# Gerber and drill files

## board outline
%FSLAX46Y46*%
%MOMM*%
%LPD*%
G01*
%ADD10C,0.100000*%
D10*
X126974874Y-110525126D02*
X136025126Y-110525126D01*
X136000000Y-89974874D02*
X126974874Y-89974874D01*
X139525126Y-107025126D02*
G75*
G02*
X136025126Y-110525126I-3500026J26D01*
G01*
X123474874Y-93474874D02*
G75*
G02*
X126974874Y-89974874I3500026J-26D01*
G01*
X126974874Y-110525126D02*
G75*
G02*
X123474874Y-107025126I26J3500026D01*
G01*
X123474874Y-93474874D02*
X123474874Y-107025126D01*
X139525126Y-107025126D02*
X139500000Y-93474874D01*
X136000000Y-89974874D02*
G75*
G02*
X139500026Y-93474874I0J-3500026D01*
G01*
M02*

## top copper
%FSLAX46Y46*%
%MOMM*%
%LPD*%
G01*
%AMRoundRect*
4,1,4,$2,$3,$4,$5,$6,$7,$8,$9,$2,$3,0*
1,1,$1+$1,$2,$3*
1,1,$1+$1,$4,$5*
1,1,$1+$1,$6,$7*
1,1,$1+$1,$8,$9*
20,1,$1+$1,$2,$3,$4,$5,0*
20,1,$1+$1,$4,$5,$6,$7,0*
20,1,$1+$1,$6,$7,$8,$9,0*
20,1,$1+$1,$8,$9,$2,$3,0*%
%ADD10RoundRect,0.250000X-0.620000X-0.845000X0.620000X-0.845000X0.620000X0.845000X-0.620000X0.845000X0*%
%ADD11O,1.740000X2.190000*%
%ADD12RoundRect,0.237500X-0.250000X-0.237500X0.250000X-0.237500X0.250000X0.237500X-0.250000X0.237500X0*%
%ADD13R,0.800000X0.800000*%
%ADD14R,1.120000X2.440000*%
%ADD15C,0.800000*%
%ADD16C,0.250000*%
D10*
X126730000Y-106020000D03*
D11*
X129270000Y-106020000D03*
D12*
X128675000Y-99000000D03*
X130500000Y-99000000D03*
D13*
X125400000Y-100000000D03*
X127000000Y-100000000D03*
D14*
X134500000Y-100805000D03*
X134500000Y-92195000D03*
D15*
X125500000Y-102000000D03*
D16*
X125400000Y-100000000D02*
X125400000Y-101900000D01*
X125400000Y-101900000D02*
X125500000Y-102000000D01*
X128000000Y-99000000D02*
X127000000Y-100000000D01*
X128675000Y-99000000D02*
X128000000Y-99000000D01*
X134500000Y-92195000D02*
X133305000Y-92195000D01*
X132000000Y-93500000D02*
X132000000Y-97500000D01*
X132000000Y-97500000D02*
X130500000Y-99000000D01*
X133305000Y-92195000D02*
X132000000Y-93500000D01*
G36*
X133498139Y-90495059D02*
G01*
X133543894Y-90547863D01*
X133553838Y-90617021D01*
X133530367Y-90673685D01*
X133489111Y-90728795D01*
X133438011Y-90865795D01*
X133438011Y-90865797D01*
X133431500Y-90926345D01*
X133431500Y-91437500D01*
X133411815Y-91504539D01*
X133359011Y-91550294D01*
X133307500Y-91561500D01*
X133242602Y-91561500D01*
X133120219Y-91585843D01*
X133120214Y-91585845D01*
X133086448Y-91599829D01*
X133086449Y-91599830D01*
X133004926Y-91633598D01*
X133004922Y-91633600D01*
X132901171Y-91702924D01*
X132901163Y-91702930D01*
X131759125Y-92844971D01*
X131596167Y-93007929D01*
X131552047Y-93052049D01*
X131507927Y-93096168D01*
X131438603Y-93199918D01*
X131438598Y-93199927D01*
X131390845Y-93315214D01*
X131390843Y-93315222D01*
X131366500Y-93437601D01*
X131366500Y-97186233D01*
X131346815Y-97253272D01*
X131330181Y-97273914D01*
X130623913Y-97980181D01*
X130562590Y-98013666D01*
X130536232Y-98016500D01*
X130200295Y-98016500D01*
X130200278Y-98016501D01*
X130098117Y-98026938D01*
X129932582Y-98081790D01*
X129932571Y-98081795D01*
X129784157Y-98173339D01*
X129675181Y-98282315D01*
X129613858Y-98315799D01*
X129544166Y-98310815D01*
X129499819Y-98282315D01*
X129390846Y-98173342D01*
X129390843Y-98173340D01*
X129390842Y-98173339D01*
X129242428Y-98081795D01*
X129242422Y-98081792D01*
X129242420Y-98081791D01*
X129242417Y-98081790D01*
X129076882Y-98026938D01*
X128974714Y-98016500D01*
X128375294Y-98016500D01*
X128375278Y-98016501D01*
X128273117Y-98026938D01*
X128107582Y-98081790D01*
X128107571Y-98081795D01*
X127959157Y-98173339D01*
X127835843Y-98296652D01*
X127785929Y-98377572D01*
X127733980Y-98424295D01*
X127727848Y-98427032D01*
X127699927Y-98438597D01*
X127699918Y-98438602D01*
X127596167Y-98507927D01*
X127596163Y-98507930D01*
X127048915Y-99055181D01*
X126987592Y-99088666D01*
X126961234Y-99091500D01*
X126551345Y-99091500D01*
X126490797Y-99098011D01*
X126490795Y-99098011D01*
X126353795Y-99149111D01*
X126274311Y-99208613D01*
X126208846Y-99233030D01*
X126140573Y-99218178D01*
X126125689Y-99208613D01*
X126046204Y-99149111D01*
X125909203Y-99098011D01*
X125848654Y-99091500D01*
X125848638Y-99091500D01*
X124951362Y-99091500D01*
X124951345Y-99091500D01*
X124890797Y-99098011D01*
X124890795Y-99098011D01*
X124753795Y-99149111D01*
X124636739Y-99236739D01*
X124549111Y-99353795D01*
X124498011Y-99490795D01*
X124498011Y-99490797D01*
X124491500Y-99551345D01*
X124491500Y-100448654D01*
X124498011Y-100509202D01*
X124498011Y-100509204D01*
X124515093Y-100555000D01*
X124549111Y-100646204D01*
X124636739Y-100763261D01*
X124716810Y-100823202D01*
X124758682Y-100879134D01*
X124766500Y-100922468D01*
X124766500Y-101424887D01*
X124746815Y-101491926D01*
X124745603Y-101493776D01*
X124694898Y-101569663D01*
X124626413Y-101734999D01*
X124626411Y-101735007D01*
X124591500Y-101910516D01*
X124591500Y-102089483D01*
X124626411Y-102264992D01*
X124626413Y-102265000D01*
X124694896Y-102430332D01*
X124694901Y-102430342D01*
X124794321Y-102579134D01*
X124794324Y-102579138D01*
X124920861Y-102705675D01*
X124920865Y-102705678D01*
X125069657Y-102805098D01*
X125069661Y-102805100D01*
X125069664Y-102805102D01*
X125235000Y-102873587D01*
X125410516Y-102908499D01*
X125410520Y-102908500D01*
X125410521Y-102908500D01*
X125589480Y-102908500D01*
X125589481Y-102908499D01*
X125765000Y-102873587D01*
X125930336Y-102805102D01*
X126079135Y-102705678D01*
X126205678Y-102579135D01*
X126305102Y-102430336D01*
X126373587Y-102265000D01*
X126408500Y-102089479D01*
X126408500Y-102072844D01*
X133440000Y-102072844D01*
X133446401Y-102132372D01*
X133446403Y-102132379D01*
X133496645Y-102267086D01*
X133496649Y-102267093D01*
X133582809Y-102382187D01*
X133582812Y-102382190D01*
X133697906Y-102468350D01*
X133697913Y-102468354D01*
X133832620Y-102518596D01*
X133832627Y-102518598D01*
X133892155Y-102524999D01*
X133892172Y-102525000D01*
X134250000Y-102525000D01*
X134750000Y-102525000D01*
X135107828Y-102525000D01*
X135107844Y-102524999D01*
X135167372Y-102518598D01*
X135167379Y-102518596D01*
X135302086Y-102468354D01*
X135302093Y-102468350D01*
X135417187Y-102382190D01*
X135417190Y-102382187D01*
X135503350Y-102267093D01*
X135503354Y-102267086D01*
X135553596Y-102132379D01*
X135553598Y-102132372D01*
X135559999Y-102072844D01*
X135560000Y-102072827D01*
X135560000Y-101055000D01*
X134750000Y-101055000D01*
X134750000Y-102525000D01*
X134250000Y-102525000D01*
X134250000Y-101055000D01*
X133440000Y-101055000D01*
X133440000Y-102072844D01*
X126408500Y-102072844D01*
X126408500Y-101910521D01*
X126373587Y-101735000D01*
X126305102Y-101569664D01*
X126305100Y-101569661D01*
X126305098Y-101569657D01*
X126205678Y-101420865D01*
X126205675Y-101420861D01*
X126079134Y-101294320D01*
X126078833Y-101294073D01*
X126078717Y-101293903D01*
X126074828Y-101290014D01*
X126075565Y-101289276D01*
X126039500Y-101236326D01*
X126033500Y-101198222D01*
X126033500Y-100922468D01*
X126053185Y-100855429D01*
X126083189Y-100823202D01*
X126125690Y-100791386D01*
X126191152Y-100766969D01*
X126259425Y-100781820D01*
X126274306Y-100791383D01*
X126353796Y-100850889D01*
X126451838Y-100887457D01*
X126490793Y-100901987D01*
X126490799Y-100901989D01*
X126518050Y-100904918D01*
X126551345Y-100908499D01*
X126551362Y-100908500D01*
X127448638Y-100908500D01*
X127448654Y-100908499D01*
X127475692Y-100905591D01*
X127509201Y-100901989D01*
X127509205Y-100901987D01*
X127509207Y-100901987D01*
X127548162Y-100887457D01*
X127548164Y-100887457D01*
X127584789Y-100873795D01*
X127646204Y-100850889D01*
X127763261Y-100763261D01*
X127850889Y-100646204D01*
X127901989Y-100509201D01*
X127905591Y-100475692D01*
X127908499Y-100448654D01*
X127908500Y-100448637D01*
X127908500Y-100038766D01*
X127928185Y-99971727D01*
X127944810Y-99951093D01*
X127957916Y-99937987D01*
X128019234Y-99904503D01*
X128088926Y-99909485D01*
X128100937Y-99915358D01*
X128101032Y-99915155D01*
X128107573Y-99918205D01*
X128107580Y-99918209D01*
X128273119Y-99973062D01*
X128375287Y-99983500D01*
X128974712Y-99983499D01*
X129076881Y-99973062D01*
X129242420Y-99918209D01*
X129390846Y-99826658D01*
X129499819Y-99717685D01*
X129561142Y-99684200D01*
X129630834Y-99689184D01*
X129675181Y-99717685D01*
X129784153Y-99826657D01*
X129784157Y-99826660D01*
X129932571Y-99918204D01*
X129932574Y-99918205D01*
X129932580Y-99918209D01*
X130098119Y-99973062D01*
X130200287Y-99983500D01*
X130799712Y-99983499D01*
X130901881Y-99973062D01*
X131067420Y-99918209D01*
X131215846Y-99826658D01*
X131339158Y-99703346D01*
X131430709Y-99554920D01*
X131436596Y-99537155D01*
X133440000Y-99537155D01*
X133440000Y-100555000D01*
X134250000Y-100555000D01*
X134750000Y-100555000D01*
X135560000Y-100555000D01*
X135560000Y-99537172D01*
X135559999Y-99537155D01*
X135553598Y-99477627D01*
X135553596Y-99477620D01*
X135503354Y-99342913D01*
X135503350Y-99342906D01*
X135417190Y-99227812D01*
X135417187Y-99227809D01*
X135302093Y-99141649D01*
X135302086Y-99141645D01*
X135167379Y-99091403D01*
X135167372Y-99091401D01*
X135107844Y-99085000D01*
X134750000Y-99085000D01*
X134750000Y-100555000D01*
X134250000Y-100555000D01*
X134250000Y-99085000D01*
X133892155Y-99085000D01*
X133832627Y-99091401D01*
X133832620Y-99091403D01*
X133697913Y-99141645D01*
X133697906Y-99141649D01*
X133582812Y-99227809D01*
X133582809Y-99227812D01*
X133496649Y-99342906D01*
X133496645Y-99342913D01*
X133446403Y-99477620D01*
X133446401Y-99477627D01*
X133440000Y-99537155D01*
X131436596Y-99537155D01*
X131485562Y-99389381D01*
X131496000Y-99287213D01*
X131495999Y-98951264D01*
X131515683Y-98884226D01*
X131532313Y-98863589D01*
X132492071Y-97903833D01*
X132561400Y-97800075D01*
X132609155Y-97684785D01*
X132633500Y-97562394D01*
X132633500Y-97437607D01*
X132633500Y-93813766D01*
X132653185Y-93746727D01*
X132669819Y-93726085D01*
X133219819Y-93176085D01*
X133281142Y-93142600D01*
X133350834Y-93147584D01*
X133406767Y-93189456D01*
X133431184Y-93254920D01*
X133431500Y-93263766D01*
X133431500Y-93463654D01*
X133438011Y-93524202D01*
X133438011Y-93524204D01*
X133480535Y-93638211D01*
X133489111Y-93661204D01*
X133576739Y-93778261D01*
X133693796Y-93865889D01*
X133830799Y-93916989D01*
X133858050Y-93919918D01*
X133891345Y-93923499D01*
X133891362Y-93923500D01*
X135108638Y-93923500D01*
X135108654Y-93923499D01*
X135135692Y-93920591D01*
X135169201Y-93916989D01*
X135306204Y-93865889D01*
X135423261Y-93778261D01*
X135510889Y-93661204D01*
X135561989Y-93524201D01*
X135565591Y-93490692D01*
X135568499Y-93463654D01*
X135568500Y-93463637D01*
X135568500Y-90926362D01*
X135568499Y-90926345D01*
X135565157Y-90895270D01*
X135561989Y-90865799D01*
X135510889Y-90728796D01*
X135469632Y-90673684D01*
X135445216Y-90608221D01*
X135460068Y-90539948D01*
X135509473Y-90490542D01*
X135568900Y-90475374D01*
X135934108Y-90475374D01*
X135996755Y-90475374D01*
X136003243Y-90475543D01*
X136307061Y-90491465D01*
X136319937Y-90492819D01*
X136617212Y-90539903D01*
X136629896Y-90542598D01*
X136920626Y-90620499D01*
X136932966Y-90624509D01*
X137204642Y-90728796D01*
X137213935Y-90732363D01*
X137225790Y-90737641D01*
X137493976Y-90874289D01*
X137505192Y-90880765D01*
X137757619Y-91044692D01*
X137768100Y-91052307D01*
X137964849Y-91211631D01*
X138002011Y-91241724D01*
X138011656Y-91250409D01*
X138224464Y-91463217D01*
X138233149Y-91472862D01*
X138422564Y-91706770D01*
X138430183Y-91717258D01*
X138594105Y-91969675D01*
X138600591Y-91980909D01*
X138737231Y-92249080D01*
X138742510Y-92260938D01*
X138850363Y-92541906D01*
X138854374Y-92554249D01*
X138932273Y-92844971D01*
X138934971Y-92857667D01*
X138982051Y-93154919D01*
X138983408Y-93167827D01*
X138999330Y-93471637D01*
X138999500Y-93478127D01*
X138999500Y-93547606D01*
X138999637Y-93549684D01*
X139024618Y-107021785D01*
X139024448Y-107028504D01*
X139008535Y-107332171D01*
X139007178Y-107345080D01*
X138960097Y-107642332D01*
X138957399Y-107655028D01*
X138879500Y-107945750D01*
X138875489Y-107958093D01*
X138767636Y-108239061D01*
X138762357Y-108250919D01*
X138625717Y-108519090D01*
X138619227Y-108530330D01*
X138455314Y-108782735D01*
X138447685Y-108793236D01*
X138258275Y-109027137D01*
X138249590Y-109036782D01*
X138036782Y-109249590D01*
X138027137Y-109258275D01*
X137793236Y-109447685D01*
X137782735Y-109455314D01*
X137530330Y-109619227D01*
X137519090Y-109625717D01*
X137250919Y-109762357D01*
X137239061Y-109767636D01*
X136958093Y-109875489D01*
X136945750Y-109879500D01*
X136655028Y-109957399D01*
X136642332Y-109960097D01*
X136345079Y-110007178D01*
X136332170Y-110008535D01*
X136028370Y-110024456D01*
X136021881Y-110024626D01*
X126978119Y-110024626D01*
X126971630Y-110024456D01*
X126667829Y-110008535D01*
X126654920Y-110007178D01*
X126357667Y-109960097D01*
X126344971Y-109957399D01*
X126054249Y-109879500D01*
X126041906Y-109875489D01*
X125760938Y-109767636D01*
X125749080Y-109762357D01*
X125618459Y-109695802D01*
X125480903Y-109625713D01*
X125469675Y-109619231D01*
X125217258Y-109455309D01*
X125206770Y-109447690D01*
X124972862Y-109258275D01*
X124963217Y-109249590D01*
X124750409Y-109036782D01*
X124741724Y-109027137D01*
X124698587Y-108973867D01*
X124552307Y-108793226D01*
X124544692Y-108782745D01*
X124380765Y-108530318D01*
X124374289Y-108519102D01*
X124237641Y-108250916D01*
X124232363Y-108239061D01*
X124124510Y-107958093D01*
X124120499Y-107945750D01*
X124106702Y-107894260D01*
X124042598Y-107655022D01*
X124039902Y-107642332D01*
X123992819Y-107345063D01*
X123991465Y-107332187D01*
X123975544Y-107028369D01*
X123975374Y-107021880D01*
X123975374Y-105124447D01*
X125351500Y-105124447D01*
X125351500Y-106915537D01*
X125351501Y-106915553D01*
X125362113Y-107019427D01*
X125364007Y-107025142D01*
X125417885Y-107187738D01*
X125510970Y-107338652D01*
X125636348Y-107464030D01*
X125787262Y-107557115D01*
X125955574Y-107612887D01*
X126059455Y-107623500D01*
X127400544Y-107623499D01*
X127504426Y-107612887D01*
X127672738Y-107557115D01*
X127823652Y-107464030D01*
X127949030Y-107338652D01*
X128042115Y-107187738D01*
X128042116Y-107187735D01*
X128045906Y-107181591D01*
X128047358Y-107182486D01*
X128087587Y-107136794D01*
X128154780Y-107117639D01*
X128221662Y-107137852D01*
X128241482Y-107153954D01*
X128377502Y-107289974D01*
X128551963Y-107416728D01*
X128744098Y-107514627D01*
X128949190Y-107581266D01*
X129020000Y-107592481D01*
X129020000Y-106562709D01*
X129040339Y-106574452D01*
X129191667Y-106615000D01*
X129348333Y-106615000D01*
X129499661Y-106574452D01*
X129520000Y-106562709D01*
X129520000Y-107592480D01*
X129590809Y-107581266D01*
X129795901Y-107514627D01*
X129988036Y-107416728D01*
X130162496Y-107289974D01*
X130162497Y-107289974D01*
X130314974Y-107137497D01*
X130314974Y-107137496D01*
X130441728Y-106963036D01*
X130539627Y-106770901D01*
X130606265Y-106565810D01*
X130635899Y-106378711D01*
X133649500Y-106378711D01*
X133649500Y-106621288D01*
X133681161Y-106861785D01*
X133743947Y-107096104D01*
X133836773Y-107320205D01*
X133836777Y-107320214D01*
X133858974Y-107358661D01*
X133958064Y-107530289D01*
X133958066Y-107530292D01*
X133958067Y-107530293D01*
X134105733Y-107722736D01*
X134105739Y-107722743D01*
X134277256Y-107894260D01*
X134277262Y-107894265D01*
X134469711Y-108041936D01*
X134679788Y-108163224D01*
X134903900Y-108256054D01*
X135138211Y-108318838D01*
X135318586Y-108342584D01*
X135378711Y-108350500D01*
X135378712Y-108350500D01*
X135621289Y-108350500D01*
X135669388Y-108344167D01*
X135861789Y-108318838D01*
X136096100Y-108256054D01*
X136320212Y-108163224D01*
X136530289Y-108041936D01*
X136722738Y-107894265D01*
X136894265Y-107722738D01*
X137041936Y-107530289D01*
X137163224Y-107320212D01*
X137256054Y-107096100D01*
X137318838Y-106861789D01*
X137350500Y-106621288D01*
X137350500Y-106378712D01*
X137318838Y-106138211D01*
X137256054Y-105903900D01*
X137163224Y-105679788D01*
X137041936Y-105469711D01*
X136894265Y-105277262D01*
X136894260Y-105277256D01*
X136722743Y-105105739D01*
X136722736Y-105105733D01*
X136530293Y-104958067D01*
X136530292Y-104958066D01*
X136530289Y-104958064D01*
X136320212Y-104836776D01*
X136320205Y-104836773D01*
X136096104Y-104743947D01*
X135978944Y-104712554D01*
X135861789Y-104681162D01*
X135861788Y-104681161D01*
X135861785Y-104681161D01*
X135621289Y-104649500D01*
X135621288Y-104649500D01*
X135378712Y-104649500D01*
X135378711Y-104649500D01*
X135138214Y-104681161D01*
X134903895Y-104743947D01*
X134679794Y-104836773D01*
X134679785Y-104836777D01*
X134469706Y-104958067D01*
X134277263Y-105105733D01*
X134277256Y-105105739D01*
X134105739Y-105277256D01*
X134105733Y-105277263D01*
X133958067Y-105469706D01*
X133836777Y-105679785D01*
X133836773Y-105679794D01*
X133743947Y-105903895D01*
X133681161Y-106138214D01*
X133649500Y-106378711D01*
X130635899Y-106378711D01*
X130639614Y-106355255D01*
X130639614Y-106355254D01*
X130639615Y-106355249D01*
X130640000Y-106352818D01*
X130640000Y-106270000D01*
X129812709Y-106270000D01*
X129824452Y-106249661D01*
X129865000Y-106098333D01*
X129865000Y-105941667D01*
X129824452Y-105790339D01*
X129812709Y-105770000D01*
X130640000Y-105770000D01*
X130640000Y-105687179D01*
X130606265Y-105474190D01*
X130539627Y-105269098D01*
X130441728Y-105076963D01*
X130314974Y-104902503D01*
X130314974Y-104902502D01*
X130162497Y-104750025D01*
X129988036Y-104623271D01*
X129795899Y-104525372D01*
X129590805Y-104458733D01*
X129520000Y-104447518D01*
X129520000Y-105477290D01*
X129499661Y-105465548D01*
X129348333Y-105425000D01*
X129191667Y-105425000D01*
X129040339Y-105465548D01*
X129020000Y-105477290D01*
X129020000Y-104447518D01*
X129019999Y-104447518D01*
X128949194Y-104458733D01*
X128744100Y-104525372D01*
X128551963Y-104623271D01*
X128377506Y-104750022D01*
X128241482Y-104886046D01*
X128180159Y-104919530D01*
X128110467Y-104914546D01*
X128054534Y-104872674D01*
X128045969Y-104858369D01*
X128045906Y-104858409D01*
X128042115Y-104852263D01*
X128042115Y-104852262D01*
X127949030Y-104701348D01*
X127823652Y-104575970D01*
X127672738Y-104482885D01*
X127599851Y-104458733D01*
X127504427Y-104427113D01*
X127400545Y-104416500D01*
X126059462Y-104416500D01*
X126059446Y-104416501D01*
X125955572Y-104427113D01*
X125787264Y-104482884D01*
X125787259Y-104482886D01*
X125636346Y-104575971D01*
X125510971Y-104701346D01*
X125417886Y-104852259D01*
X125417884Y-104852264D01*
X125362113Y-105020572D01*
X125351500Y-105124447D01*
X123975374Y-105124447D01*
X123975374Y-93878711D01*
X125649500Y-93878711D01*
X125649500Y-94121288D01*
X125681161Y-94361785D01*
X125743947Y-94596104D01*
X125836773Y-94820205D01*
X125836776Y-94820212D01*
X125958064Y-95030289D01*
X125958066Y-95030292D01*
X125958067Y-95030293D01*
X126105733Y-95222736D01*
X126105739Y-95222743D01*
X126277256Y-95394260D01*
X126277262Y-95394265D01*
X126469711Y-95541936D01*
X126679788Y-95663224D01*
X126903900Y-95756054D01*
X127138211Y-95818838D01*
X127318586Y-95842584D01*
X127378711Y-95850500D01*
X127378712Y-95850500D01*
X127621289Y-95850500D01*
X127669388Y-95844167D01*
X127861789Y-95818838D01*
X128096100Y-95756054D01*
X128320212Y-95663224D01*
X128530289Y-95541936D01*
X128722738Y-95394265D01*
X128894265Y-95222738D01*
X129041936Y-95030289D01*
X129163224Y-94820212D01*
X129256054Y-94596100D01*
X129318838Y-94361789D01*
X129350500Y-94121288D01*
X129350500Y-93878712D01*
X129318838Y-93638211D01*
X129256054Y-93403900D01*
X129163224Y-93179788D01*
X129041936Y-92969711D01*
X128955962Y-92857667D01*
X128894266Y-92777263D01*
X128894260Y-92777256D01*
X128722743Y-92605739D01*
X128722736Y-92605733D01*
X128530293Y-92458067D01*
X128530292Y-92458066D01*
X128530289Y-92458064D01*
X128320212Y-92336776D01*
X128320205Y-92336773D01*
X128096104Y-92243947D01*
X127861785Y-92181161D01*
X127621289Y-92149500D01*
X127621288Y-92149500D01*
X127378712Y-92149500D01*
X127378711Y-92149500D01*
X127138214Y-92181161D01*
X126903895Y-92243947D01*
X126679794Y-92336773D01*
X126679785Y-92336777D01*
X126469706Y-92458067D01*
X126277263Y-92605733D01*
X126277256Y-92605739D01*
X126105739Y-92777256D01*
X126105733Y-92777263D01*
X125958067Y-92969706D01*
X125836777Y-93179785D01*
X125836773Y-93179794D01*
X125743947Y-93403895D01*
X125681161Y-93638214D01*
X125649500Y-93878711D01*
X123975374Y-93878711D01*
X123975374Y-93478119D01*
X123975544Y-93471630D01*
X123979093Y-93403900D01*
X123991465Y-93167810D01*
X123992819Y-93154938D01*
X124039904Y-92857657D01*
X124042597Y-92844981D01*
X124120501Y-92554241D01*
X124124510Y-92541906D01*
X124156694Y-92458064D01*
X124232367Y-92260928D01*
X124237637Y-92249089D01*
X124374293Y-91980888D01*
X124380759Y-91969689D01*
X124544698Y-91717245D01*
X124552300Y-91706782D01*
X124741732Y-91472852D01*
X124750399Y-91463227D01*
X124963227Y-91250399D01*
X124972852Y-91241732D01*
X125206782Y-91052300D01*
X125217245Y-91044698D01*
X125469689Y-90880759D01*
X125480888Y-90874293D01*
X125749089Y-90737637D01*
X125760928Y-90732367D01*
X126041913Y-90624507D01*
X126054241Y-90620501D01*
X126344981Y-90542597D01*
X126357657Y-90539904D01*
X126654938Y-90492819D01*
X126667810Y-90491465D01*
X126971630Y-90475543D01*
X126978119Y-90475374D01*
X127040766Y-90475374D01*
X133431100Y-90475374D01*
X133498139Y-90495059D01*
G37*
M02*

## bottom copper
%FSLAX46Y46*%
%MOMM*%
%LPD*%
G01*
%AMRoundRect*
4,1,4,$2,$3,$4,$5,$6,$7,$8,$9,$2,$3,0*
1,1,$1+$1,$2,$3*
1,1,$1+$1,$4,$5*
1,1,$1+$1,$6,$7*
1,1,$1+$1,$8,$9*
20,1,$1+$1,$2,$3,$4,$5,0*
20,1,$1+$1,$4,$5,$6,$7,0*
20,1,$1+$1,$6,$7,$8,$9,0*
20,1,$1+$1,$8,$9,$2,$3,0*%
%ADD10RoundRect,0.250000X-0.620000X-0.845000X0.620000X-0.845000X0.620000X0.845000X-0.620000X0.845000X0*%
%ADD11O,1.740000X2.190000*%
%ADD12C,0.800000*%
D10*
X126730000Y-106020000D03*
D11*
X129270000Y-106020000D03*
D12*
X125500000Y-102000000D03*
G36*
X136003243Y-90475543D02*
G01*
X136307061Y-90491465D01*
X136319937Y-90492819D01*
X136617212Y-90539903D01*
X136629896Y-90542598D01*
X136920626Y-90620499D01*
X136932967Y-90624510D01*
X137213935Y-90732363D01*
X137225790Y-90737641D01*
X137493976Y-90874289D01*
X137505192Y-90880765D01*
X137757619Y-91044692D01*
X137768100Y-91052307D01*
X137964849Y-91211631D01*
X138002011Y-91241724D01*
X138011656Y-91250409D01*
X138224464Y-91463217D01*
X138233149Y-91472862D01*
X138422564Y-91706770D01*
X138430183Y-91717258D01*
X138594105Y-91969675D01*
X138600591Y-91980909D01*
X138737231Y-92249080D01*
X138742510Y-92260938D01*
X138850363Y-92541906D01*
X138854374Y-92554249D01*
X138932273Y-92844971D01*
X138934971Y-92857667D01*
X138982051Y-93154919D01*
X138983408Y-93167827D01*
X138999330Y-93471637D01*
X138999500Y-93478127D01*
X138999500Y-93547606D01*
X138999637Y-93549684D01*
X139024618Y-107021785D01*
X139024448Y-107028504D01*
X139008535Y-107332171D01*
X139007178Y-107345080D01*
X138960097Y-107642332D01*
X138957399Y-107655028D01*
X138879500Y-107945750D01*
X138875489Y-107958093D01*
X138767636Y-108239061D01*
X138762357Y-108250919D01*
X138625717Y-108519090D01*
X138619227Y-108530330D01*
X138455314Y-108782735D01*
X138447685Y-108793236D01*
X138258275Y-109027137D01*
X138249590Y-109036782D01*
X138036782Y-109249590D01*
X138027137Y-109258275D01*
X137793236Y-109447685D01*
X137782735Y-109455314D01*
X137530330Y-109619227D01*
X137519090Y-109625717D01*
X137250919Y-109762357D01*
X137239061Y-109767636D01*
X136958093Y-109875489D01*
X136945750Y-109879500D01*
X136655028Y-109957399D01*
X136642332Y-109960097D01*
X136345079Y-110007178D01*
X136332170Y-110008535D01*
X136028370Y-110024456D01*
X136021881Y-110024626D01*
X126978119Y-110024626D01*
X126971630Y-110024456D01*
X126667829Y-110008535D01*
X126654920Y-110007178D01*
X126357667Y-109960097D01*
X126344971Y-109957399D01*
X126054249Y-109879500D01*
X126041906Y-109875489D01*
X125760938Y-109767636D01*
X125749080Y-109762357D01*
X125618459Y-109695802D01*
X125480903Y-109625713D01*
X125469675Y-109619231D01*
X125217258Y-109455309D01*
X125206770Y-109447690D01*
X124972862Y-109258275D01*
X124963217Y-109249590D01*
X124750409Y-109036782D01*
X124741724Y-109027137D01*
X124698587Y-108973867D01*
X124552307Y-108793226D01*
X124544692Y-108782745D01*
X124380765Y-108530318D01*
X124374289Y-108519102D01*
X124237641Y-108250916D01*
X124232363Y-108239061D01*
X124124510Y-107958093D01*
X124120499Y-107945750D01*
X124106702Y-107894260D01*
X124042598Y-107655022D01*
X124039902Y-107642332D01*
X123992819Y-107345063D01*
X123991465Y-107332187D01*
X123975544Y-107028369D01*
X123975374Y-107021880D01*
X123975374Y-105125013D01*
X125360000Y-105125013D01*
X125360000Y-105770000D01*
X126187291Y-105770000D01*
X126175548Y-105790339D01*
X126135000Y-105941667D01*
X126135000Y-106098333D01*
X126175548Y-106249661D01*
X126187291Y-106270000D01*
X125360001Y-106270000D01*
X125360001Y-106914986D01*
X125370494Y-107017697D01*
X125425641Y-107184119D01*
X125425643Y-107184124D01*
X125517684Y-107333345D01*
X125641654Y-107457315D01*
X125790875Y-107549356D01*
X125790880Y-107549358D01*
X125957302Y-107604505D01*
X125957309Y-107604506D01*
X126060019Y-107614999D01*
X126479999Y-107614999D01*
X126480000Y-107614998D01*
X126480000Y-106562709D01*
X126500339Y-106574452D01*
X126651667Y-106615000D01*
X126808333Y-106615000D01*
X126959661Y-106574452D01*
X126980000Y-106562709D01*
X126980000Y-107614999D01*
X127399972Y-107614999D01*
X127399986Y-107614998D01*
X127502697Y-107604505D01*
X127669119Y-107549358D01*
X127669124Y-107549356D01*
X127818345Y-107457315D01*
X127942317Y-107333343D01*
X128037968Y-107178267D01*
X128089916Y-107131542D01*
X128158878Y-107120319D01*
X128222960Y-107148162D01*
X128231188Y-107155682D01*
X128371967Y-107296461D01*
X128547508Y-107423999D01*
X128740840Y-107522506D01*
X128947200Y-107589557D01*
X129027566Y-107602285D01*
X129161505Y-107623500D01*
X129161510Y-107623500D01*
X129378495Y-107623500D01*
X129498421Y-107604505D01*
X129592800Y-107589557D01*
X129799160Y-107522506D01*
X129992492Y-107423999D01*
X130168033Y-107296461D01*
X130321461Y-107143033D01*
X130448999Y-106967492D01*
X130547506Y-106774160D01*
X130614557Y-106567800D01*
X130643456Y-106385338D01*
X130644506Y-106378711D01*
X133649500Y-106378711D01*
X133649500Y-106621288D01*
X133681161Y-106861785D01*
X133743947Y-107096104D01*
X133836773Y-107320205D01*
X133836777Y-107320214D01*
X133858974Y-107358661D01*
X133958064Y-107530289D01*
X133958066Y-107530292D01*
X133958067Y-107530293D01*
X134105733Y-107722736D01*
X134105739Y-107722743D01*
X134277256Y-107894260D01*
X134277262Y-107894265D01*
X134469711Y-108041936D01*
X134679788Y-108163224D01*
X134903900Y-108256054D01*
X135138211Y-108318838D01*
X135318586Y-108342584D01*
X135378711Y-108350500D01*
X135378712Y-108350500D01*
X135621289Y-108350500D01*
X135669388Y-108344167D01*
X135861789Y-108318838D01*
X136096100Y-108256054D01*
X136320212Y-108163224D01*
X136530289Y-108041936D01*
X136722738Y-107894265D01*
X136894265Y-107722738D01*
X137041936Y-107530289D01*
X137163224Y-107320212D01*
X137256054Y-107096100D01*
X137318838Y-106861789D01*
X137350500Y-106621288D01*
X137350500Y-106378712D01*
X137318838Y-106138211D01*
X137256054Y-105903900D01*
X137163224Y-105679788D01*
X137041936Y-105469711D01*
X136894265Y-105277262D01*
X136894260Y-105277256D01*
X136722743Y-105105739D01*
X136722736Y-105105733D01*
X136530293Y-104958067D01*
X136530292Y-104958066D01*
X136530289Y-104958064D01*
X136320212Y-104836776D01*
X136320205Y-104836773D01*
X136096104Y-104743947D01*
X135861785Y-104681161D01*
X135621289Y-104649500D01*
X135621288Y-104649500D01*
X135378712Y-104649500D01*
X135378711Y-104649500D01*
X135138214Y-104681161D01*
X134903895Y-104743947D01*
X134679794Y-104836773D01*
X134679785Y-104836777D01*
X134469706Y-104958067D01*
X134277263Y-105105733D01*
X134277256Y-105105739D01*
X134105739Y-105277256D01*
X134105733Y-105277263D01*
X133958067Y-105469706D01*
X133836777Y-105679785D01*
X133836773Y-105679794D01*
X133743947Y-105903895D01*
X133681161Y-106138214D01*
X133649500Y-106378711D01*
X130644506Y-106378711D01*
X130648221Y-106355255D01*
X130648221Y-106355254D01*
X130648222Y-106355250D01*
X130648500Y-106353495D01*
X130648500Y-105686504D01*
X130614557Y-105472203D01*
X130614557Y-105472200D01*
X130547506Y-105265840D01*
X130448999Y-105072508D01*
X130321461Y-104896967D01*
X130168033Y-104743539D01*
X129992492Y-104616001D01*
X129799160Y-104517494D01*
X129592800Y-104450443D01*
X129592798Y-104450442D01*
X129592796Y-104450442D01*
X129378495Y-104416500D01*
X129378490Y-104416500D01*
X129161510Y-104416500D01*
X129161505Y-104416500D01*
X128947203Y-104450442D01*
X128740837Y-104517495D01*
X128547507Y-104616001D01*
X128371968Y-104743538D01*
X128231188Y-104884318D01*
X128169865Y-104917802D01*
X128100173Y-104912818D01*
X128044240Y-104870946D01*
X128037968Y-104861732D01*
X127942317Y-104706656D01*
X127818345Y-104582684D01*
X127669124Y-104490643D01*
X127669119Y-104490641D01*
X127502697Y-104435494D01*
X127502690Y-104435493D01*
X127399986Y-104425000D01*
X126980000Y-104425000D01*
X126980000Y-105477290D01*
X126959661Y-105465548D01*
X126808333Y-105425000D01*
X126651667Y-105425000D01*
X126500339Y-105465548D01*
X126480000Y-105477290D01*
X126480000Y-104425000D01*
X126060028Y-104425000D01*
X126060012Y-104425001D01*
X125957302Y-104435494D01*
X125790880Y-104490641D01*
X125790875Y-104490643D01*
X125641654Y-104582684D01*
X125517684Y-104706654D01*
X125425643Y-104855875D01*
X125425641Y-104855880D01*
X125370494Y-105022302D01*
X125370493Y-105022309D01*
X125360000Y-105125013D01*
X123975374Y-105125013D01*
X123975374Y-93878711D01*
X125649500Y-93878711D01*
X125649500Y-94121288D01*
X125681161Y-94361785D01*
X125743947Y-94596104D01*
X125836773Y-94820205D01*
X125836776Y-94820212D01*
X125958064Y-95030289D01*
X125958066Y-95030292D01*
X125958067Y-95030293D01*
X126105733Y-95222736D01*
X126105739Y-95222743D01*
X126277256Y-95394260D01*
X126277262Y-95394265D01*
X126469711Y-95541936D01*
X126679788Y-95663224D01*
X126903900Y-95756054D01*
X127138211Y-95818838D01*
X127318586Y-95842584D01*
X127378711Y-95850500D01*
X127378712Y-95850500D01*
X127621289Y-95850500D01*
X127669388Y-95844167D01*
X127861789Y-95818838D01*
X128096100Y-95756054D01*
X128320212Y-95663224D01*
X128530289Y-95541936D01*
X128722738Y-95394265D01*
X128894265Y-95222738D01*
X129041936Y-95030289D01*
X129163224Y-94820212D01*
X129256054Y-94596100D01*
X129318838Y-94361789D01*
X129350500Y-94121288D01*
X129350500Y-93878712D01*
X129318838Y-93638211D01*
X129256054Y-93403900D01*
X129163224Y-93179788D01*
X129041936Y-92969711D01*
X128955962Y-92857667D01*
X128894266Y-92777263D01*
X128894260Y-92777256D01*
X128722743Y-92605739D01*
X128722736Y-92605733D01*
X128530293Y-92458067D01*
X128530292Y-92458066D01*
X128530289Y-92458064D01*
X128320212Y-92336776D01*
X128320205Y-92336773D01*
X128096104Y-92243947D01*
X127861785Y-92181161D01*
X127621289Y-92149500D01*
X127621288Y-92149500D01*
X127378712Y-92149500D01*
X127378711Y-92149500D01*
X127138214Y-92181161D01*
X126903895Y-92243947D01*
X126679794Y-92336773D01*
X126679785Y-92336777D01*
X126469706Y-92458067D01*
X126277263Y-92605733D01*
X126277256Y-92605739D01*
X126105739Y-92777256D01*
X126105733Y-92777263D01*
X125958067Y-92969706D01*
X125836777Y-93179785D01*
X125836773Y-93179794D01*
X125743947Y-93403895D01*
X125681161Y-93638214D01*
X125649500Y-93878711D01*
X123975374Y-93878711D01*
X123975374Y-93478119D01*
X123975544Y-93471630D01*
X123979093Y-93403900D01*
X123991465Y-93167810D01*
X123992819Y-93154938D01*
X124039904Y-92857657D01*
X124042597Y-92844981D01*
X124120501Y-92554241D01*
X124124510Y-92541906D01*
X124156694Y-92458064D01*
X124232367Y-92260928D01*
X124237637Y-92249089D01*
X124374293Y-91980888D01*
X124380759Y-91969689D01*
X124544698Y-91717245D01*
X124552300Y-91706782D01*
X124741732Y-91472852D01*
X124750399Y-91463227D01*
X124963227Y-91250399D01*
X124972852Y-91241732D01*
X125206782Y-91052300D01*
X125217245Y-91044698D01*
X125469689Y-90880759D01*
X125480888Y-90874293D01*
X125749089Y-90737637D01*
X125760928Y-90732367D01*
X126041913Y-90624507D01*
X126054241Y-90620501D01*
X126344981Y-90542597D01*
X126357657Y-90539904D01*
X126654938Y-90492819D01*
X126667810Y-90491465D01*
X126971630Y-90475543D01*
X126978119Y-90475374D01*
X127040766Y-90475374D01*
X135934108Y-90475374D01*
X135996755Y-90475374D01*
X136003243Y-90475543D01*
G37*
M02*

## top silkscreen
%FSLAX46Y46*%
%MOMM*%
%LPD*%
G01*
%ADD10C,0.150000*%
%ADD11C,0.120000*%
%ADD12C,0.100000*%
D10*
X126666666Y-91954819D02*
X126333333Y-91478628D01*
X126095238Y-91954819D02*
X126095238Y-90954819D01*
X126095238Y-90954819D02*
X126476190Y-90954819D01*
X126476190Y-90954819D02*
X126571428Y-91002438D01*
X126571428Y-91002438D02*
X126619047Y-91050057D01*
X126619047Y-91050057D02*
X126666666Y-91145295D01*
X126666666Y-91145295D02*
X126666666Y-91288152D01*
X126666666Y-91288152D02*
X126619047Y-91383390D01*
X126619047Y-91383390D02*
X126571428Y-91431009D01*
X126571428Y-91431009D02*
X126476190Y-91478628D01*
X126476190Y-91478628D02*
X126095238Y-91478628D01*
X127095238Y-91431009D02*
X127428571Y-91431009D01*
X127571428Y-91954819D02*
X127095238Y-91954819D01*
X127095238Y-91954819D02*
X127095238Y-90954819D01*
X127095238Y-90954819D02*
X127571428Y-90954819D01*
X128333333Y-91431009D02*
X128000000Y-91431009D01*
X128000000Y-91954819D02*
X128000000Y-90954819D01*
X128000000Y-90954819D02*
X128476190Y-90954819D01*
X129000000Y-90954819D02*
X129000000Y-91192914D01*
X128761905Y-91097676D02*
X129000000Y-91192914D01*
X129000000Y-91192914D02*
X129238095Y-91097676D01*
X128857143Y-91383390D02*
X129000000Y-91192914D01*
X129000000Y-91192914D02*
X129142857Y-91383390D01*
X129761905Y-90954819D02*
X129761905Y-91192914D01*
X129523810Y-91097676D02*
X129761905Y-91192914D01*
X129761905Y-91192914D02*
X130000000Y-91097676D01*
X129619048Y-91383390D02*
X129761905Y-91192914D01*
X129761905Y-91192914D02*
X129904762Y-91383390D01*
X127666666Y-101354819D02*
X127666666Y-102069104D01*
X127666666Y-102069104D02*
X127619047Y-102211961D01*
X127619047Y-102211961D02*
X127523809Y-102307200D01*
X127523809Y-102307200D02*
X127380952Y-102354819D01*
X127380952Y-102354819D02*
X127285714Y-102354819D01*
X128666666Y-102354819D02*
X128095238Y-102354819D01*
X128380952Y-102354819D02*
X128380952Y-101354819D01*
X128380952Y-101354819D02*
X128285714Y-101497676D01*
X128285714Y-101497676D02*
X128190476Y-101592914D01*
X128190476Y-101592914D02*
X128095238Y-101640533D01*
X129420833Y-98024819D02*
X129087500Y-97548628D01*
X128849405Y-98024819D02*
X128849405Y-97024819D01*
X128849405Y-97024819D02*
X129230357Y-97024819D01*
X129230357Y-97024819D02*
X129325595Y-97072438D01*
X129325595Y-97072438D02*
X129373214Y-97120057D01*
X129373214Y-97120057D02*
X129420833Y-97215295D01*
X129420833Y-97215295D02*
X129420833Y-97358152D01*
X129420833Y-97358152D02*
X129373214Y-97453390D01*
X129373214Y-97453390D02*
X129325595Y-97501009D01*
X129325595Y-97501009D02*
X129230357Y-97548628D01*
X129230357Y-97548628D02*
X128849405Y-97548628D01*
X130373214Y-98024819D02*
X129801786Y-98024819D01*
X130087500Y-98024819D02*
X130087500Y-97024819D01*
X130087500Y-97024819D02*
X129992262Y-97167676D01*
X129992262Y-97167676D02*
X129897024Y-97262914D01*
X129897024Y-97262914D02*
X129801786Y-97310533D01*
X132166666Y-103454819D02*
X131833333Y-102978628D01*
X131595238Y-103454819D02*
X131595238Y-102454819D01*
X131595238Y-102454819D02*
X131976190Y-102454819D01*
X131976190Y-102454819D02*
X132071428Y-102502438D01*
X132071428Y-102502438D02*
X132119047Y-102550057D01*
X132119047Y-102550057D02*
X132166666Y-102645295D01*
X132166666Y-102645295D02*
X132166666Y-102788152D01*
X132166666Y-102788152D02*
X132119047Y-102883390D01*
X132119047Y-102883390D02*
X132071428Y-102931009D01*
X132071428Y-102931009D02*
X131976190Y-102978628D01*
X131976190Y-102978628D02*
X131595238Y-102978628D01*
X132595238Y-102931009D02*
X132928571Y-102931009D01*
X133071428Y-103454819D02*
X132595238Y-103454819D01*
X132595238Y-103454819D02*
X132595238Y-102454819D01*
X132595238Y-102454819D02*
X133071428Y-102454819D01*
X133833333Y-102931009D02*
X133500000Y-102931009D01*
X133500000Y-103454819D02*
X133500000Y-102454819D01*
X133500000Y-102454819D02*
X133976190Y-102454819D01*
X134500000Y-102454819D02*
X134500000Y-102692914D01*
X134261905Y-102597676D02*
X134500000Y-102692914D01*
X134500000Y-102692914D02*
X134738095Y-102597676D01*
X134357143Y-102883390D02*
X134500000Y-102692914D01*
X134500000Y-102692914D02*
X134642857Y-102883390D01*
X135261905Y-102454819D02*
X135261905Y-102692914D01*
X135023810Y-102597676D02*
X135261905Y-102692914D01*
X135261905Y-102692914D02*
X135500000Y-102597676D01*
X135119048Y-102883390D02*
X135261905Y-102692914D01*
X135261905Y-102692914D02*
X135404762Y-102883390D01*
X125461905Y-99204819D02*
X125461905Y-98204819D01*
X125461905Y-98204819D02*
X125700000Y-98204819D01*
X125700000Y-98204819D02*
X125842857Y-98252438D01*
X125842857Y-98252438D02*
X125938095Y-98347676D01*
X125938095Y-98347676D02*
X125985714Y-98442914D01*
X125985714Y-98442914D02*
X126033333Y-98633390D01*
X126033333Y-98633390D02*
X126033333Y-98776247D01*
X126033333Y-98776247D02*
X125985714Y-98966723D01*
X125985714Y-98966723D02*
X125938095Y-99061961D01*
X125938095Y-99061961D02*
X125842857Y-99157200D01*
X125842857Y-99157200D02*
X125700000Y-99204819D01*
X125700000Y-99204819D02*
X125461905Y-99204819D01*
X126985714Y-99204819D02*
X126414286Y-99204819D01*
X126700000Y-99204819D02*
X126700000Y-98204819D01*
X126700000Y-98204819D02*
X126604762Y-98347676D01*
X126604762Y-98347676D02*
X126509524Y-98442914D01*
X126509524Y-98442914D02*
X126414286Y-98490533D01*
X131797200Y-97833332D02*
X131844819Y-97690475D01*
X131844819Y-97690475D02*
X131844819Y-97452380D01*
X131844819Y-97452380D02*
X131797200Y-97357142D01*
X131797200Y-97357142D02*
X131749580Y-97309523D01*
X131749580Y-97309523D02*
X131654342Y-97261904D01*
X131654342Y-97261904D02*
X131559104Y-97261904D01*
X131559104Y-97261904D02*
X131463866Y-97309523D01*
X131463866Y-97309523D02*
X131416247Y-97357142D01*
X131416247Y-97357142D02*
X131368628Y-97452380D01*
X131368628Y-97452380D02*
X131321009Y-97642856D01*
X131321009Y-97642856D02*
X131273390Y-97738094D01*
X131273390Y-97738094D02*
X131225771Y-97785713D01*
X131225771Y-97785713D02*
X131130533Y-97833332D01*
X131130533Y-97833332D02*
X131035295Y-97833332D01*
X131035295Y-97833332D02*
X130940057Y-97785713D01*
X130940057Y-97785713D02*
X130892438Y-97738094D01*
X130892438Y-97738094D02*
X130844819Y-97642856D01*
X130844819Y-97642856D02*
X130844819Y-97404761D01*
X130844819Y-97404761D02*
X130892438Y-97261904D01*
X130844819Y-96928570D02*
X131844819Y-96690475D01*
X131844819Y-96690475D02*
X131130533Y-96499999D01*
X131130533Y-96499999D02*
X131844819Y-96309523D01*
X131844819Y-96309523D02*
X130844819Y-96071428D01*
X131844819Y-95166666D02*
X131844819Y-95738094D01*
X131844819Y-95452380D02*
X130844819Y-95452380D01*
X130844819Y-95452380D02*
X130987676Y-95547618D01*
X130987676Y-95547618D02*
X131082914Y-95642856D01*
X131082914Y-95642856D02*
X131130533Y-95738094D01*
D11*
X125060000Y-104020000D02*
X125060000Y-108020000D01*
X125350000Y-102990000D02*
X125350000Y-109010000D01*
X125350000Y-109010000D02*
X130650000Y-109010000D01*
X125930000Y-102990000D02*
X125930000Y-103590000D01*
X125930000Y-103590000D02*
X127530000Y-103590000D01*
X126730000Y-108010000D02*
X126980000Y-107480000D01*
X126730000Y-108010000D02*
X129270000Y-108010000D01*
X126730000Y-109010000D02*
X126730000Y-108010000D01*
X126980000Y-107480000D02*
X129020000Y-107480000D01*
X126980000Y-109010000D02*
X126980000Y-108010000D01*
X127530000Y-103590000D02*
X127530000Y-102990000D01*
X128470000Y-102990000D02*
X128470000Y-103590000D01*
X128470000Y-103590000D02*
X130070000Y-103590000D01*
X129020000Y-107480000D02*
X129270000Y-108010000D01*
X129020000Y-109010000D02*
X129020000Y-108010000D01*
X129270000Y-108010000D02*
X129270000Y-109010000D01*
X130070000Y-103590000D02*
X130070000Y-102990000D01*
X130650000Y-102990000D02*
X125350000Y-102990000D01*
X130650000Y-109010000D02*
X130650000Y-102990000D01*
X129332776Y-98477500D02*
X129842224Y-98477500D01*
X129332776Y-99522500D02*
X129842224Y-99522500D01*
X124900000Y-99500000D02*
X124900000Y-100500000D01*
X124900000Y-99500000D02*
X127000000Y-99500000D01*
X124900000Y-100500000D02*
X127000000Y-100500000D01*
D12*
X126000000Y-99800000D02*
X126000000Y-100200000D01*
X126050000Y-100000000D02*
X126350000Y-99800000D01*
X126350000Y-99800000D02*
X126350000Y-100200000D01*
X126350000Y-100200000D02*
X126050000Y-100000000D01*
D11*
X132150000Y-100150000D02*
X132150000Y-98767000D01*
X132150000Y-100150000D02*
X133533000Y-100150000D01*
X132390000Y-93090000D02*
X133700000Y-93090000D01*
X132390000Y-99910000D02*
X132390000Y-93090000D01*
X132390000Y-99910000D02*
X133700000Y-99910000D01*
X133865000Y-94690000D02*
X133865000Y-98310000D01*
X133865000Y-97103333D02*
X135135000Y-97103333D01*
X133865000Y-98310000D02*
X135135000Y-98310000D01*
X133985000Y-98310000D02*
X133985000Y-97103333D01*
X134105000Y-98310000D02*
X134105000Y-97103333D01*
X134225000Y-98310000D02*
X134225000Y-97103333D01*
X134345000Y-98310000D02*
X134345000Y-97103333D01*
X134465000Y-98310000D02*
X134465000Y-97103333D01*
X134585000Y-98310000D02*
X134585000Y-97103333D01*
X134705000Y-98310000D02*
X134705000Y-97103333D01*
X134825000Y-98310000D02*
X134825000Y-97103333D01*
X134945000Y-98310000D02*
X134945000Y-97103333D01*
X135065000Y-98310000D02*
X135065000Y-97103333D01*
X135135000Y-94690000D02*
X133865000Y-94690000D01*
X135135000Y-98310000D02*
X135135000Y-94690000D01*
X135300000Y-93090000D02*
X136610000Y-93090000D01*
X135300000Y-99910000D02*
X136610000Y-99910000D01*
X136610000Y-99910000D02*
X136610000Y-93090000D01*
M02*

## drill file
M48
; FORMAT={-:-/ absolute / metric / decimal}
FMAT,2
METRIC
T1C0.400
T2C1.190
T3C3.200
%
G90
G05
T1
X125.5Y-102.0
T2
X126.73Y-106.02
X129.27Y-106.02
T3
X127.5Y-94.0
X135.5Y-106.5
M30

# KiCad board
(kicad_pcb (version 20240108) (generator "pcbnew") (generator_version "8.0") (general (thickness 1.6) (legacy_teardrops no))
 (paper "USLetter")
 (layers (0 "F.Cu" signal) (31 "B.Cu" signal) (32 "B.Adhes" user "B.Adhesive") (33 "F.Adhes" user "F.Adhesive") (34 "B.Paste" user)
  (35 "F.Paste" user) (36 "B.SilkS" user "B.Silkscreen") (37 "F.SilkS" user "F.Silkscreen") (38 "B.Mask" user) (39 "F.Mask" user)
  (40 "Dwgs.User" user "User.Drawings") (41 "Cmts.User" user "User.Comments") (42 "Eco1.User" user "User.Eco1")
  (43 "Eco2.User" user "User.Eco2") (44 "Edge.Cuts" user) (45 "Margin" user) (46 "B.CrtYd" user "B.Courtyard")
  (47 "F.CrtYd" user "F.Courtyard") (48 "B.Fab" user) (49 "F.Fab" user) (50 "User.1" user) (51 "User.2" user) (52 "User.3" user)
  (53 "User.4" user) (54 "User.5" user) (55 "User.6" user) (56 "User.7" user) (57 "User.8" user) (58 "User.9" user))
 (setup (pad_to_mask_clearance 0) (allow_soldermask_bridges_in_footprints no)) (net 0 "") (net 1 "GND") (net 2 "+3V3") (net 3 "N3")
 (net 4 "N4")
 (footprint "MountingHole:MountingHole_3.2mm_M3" (layer "F.Cu") (at 127.5 94)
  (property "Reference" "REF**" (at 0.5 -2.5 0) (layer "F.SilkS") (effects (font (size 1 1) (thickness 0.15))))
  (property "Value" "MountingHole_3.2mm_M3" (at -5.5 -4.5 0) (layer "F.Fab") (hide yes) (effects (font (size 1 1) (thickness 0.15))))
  (pad "" np_thru_hole circle (at 0 0) (size 3.2 3.2) (drill 3.2) (layers "*.Cu" "*.Mask")))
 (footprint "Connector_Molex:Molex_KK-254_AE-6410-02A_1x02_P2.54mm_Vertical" (layer "F.Cu") (at 126.73 106.02)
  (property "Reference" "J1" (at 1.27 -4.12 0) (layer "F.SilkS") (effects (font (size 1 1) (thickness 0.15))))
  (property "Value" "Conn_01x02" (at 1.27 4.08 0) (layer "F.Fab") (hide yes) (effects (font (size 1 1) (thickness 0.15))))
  (fp_line (start -1.67 -2) (end -1.67 2) (stroke (width 0.12) (type solid)) (layer "F.SilkS"))
  (fp_line (start -1.38 -3.03) (end -1.38 2.99) (stroke (width 0.12) (type solid)) (layer "F.SilkS"))
  (fp_line (start -1.38 2.99) (end 3.92 2.99) (stroke (width 0.12) (type solid)) (layer "F.SilkS"))
  (fp_line (start -0.8 -3.03) (end -0.8 -2.43) (stroke (width 0.12) (type solid)) (layer "F.SilkS"))
  (fp_line (start -0.8 -2.43) (end 0.8 -2.43) (stroke (width 0.12) (type solid)) (layer "F.SilkS"))
  (fp_line (start 0 1.99) (end 0.25 1.46) (stroke (width 0.12) (type solid)) (layer "F.SilkS"))
  (fp_line (start 0 1.99) (end 2.54 1.99) (stroke (width 0.12) (type solid)) (layer "F.SilkS"))
  (fp_line (start 0 2.99) (end 0 1.99) (stroke (width 0.12) (type solid)) (layer "F.SilkS"))
  (fp_line (start 0.25 1.46) (end 2.29 1.46) (stroke (width 0.12) (type solid)) (layer "F.SilkS"))
  (fp_line (start 0.25 2.99) (end 0.25 1.99) (stroke (width 0.12) (type solid)) (layer "F.SilkS"))
  (fp_line (start 0.8 -2.43) (end 0.8 -3.03) (stroke (width 0.12) (type solid)) (layer "F.SilkS"))
  (fp_line (start 1.74 -3.03) (end 1.74 -2.43) (stroke (width 0.12) (type solid)) (layer "F.SilkS"))
  (fp_line (start 1.74 -2.43) (end 3.34 -2.43) (stroke (width 0.12) (type solid)) (layer "F.SilkS"))
  (fp_line (start 2.29 1.46) (end 2.54 1.99) (stroke (width 0.12) (type solid)) (layer "F.SilkS"))
  (fp_line (start 2.29 2.99) (end 2.29 1.99) (stroke (width 0.12) (type solid)) (layer "F.SilkS"))
  (fp_line (start 2.54 1.99) (end 2.54 2.99) (stroke (width 0.12) (type solid)) (layer "F.SilkS"))
  (fp_line (start 3.34 -2.43) (end 3.34 -3.03) (stroke (width 0.12) (type solid)) (layer "F.SilkS"))
  (fp_line (start 3.92 -3.03) (end -1.38 -3.03) (stroke (width 0.12) (type solid)) (layer "F.SilkS"))
  (fp_line (start 3.92 2.99) (end 3.92 -3.03) (stroke (width 0.12) (type solid)) (layer "F.SilkS"))
  (pad "1" thru_hole roundrect (at 0 0) (size 1.74 2.19) (drill 1.19) (layers "*.Cu" "*.Mask") (remove_unused_layers no)
   (roundrect_rratio 0.143678) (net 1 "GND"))
  (pad "2" thru_hole oval (at 2.54 0) (size 1.74 2.19) (drill 1.19) (layers "*.Cu" "*.Mask") (remove_unused_layers no) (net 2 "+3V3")))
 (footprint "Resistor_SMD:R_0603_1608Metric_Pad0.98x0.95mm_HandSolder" (layer "F.Cu") (at 129.5875 99)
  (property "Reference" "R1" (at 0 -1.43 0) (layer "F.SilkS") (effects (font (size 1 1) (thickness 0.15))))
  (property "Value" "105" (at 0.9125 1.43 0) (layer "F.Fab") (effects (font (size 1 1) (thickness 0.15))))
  (fp_line (start -0.254724 -0.5225) (end 0.254724 -0.5225) (stroke (width 0.12) (type solid)) (layer "F.SilkS"))
  (fp_line (start -0.254724 0.5225) (end 0.254724 0.5225) (stroke (width 0.12) (type solid)) (layer "F.SilkS"))
  (pad "1" smd roundrect (at -0.9125 0) (size 0.975 0.95) (layers "F.Cu" "F.Paste" "F.Mask") (roundrect_rratio 0.25) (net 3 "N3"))
  (pad "2" smd roundrect (at 0.9125 0) (size 0.975 0.95) (layers "F.Cu" "F.Paste" "F.Mask") (roundrect_rratio 0.25) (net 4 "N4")))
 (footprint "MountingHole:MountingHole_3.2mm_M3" (layer "F.Cu") (at 135.5 106.5)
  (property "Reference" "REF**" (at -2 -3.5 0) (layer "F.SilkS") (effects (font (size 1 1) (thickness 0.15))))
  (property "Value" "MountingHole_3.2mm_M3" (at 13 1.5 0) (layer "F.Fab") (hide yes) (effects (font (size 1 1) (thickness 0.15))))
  (pad "" np_thru_hole circle (at 0 0) (size 3.2 3.2) (drill 3.2) (layers "*.Cu" "*.Mask")))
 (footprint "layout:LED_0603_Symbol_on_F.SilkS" (layer "F.Cu") (at 126.2 100)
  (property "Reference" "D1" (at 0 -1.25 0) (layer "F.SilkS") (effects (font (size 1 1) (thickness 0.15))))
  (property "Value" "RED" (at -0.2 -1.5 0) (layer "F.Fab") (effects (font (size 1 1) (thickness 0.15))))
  (fp_line (start -1.3 -0.5) (end -1.3 0.5) (stroke (width 0.12) (type solid)) (layer "F.SilkS"))
  (fp_line (start -1.3 -0.5) (end 0.8 -0.5) (stroke (width 0.12) (type solid)) (layer "F.SilkS"))
  (fp_line (start -1.3 0.5) (end 0.8 0.5) (stroke (width 0.12) (type solid)) (layer "F.SilkS"))
  (fp_line (start -0.2 -0.2) (end -0.2 0.2) (stroke (width 0.1) (type solid)) (layer "F.SilkS"))
  (fp_line (start -0.15 0) (end 0.15 -0.2) (stroke (width 0.1) (type solid)) (layer "F.SilkS"))
  (fp_line (start 0.15 -0.2) (end 0.15 0.2) (stroke (width 0.1) (type solid)) (layer "F.SilkS"))
  (fp_line (start 0.15 0.2) (end -0.15 0) (stroke (width 0.1) (type solid)) (layer "F.SilkS"))
  (pad "1" smd rect (at -0.8 0 180) (size 0.8 0.8) (layers "F.Cu" "F.Paste" "F.Mask") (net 1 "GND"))
  (pad "2" smd rect (at 0.8 0 180) (size 0.8 0.8) (layers "F.Cu" "F.Paste" "F.Mask") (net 3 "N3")))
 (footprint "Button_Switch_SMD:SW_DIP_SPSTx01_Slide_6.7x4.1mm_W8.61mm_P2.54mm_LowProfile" (layer "F.Cu") (at 134.5 96.5 90)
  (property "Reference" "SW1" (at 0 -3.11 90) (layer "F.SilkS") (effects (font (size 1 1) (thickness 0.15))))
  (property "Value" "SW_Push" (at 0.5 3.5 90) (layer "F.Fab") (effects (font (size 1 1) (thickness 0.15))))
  (fp_line (start -3.65 -2.35) (end -2.267 -2.35) (stroke (width 0.12) (type solid)) (layer "F.SilkS"))
  (fp_line (start -3.65 -2.35) (end -3.65 -0.967) (stroke (width 0.12) (type solid)) (layer "F.SilkS"))
  (fp_line (start 3.41 -2.11) (end 3.41 -0.8) (stroke (width 0.12) (type solid)) (layer "F.SilkS"))
  (fp_line (start -3.41 -2.11) (end 3.41 -2.11) (stroke (width 0.12) (type solid)) (layer "F.SilkS"))
  (fp_line (start -3.41 -2.11) (end -3.41 -0.8) (stroke (width 0.12) (type solid)) (layer "F.SilkS"))
  (fp_line (start 1.81 -0.635) (end -1.81 -0.635) (stroke (width 0.12) (type solid)) (layer "F.SilkS"))
  (fp_line (start -0.603333 -0.635) (end -0.603333 0.635) (stroke (width 0.12) (type solid)) (layer "F.SilkS"))
  (fp_line (start -1.81 -0.635) (end -1.81 0.635) (stroke (width 0.12) (type solid)) (layer "F.SilkS"))
  (fp_line (start -1.81 -0.515) (end -0.603333 -0.515) (stroke (width 0.12) (type solid)) (layer "F.SilkS"))
  (fp_line (start -1.81 -0.395) (end -0.603333 -0.395) (stroke (width 0.12) (type solid)) (layer "F.SilkS"))
  (fp_line (start -1.81 -0.275) (end -0.603333 -0.275) (stroke (width 0.12) (type solid)) (layer "F.SilkS"))
  (fp_line (start -1.81 -0.155) (end -0.603333 -0.155) (stroke (width 0.12) (type solid)) (layer "F.SilkS"))
  (fp_line (start -1.81 -0.035) (end -0.603333 -0.035) (stroke (width 0.12) (type solid)) (layer "F.SilkS"))
  (fp_line (start -1.81 0.085) (end -0.603333 0.085) (stroke (width 0.12) (type solid)) (layer "F.SilkS"))
  (fp_line (start -1.81 0.205) (end -0.603333 0.205) (stroke (width 0.12) (type solid)) (layer "F.SilkS"))
  (fp_line (start -1.81 0.325) (end -0.603333 0.325) (stroke (width 0.12) (type solid)) (layer "F.SilkS"))
  (fp_line (start -1.81 0.445) (end -0.603333 0.445) (stroke (width 0.12) (type solid)) (layer "F.SilkS"))
  (fp_line (start -1.81 0.565) (end -0.603333 0.565) (stroke (width 0.12) (type solid)) (layer "F.SilkS"))
  (fp_line (start 1.81 0.635) (end 1.81 -0.635) (stroke (width 0.12) (type solid)) (layer "F.SilkS"))
  (fp_line (start -1.81 0.635) (end 1.81 0.635) (stroke (width 0.12) (type solid)) (layer "F.SilkS"))
  (fp_line (start 3.41 0.8) (end 3.41 2.11) (stroke (width 0.12) (type solid)) (layer "F.SilkS"))
  (fp_line (start -3.41 0.8) (end -3.41 2.11) (stroke (width 0.12) (type solid)) (layer "F.SilkS"))
  (fp_line (start -3.41 2.11) (end 3.41 2.11) (stroke (width 0.12) (type solid)) (layer "F.SilkS"))
  (pad "1" smd rect (at -4.305 0 90) (size 2.44 1.12) (layers "F.Cu" "F.Paste" "F.Mask") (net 2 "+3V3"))
  (pad "2" smd rect (at 4.305 0 90) (size 2.44 1.12) (layers "F.Cu" "F.Paste" "F.Mask") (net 4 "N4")))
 (gr_line (start 126.974874 110.525126) (end 136.025126 110.525126) (stroke (width 0.1) (type default)) (layer "Edge.Cuts"))
 (gr_line (start 136 89.974874) (end 126.974874 89.974874) (stroke (width 0.1) (type default)) (layer "Edge.Cuts"))
 (gr_arc (start 139.525126 107.025126) (mid 138.5 109.5) (end 136.025126 110.525126) (stroke (width 0.1) (type default)) (layer "Edge.Cuts"))
 (gr_arc (start 123.474874 93.474874) (mid 124.5 91) (end 126.974874 89.974874) (stroke (width 0.1) (type default)) (layer "Edge.Cuts"))
 (gr_arc (start 126.974874 110.525126) (mid 124.5 109.5) (end 123.474874 107.025126) (stroke (width 0.1) (type default)) (layer "Edge.Cuts"))
 (gr_line (start 123.474874 93.474874) (end 123.474874 107.025126) (stroke (width 0.1) (type default)) (layer "Edge.Cuts"))
 (gr_line (start 139.525126 107.025126) (end 139.5 93.474874) (stroke (width 0.1) (type default)) (layer "Edge.Cuts"))
 (gr_arc (start 136 89.974874) (mid 138.474874 91) (end 139.5 93.474874) (stroke (width 0.1) (type default)) (layer "Edge.Cuts"))
 (segment (start 125.4 100) (end 125.4 101.9) (width 0.25) (layer "F.Cu") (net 1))
 (segment (start 125.4 101.9) (end 125.5 102) (width 0.25) (layer "F.Cu") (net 1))
 (via (at 125.5 102) (size 0.8) (drill 0.4) (layers "F.Cu" "B.Cu") (free yes) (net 1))
 (segment (start 128 99) (end 127 100) (width 0.25) (layer "F.Cu") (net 3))
 (segment (start 128.675 99) (end 128 99) (width 0.25) (layer "F.Cu") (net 3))
 (segment (start 134.5 92.195) (end 133.305 92.195) (width 0.25) (layer "F.Cu") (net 4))
 (segment (start 132 93.5) (end 132 97.5) (width 0.25) (layer "F.Cu") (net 4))
 (segment (start 132 97.5) (end 130.5 99) (width 0.25) (layer "F.Cu") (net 4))
 (segment (start 133.305 92.195) (end 132 93.5) (width 0.25) (layer "F.Cu") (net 4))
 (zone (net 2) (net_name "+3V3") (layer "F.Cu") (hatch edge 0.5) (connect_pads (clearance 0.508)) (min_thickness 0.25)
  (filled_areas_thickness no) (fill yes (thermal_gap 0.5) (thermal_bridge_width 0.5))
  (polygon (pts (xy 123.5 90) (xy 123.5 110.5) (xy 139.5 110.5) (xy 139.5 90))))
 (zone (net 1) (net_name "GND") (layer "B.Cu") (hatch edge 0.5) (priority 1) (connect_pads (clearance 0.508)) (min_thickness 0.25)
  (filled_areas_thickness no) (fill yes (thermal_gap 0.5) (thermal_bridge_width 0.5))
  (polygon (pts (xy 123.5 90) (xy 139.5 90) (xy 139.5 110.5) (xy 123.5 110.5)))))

